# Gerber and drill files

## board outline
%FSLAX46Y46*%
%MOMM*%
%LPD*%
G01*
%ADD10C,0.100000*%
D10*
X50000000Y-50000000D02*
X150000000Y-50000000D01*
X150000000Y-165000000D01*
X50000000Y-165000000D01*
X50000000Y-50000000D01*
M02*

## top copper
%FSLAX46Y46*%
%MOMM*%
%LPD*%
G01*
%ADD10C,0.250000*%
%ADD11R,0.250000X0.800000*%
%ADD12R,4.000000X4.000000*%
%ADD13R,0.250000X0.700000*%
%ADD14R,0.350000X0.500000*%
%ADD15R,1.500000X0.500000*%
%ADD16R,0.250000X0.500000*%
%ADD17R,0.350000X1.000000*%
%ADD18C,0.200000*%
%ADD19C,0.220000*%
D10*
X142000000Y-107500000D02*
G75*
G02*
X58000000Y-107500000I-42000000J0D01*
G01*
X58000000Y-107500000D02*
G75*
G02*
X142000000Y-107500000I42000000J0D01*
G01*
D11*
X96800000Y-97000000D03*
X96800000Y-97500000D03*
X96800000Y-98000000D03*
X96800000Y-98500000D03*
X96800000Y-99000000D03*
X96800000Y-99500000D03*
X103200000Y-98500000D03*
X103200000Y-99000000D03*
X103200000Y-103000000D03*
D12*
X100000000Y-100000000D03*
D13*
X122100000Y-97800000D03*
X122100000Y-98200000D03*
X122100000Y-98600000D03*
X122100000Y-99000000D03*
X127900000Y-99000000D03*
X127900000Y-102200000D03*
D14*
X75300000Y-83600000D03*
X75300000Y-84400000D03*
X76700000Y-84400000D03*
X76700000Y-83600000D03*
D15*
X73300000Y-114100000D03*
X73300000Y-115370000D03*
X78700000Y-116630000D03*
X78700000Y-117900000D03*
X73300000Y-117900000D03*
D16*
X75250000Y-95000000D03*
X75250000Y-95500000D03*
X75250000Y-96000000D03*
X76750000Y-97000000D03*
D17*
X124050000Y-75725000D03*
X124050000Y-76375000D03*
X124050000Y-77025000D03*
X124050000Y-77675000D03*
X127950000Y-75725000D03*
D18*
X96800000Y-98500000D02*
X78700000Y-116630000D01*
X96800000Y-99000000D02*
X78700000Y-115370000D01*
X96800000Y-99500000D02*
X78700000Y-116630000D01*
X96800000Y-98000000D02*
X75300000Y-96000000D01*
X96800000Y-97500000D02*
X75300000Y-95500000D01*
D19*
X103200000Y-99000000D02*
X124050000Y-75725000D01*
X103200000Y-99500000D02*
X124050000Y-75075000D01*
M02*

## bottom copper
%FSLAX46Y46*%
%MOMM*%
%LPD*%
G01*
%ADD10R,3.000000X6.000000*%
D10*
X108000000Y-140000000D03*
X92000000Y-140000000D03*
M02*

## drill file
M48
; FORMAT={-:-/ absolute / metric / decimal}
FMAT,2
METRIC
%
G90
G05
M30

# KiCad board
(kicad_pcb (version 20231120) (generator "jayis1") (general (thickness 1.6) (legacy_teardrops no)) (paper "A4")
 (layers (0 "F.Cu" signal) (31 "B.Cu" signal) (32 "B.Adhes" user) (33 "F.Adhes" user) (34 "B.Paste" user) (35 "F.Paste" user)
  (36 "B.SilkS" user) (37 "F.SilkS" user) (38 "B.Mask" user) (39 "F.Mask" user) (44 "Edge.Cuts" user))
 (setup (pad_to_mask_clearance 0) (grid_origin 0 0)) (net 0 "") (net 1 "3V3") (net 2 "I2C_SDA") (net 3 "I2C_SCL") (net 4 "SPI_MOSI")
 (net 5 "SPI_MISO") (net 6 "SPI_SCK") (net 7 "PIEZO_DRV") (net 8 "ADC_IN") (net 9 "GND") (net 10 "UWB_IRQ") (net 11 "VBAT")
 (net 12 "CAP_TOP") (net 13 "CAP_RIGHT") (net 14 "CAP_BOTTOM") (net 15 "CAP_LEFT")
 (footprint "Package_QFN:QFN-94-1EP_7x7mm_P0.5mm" (layer "F.Cu") (at 100 100) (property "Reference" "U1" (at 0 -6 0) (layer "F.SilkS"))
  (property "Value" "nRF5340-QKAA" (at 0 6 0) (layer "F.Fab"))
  (pad "1" smd rect (at -3.2 -3 0) (size 0.25 0.8) (layers "F.Cu" "F.Mask" "F.Paste") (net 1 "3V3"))
  (pad "2" smd rect (at -3.2 -2.5 0) (size 0.25 0.8) (layers "F.Cu" "F.Mask" "F.Paste") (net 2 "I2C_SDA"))
  (pad "3" smd rect (at -3.2 -2.0 0) (size 0.25 0.8) (layers "F.Cu" "F.Mask" "F.Paste") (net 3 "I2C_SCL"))
  (pad "4" smd rect (at -3.2 -1.5 0) (size 0.25 0.8) (layers "F.Cu" "F.Mask" "F.Paste") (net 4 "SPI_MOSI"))
  (pad "5" smd rect (at -3.2 -1.0 0) (size 0.25 0.8) (layers "F.Cu" "F.Mask" "F.Paste") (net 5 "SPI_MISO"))
  (pad "6" smd rect (at -3.2 -0.5 0) (size 0.25 0.8) (layers "F.Cu" "F.Mask" "F.Paste") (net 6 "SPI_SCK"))
  (pad "21" smd rect (at 3.2 -1.5 180) (size 0.25 0.8) (layers "F.Cu" "F.Mask" "F.Paste") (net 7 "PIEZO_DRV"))
  (pad "22" smd rect (at 3.2 -1.0 180) (size 0.25 0.8) (layers "F.Cu" "F.Mask" "F.Paste") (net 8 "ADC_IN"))
  (pad "47" smd rect (at 3.2 3.0 180) (size 0.25 0.8) (layers "F.Cu" "F.Mask" "F.Paste") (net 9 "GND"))
  (pad "EP" smd rect (at 0 0 0) (size 4 4) (layers "F.Cu" "F.Mask") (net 9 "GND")))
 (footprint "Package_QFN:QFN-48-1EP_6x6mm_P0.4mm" (layer "F.Cu") (at 125 100) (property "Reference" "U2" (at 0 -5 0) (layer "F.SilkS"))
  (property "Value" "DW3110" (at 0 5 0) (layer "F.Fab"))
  (pad "1" smd rect (at -2.9 -2.2 0) (size 0.25 0.7) (layers "F.Cu" "F.Mask" "F.Paste") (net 1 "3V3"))
  (pad "2" smd rect (at -2.9 -1.8 0) (size 0.25 0.7) (layers "F.Cu" "F.Mask" "F.Paste") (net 4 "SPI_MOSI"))
  (pad "3" smd rect (at -2.9 -1.4 0) (size 0.25 0.7) (layers "F.Cu" "F.Mask" "F.Paste") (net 5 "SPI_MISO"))
  (pad "4" smd rect (at -2.9 -1.0 0) (size 0.25 0.7) (layers "F.Cu" "F.Mask" "F.Paste") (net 6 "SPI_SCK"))
  (pad "10" smd rect (at 2.9 -1.0 180) (size 0.25 0.7) (layers "F.Cu" "F.Mask" "F.Paste") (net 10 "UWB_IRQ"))
  (pad "48" smd rect (at 2.9 2.2 180) (size 0.25 0.7) (layers "F.Cu" "F.Mask" "F.Paste") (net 9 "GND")))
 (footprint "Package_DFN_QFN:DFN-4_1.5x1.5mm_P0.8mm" (layer "F.Cu") (at 76 84) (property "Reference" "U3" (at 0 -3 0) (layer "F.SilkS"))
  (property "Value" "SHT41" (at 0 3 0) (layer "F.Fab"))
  (pad "1" smd rect (at -0.7 -0.4 0) (size 0.35 0.5) (layers "F.Cu" "F.Mask" "F.Paste") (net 1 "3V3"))
  (pad "2" smd rect (at -0.7 0.4 0) (size 0.35 0.5) (layers "F.Cu" "F.Mask" "F.Paste") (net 2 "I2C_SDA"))
  (pad "3" smd rect (at 0.7 0.4 0) (size 0.35 0.5) (layers "F.Cu" "F.Mask" "F.Paste") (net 3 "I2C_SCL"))
  (pad "4" smd rect (at 0.7 -0.4 0) (size 0.35 0.5) (layers "F.Cu" "F.Mask" "F.Paste") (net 9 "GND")))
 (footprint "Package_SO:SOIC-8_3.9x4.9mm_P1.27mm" (layer "F.Cu") (at 76 116) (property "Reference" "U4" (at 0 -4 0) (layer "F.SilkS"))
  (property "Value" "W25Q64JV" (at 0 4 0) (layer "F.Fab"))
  (pad "1" smd rect (at -2.7 -1.9 0) (size 1.5 0.5) (layers "F.Cu" "F.Mask" "F.Paste") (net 4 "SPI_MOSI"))
  (pad "2" smd rect (at -2.7 -0.63 0) (size 1.5 0.5) (layers "F.Cu" "F.Mask" "F.Paste") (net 5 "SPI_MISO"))
  (pad "6" smd rect (at 2.7 0.63 0) (size 1.5 0.5) (layers "F.Cu" "F.Mask" "F.Paste") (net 6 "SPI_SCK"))
  (pad "8" smd rect (at 2.7 1.9 0) (size 1.5 0.5) (layers "F.Cu" "F.Mask" "F.Paste") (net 1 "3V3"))
  (pad "4" smd rect (at -2.7 1.9 0) (size 1.5 0.5) (layers "F.Cu" "F.Mask" "F.Paste") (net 9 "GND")))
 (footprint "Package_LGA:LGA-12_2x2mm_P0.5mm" (layer "F.Cu") (at 76 96) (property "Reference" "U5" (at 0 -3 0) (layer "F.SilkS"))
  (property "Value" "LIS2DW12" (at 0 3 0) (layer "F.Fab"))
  (pad "1" smd rect (at -0.75 -1.0 0) (size 0.25 0.5) (layers "F.Cu" "F.Mask" "F.Paste") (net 1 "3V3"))
  (pad "2" smd rect (at -0.75 -0.5 0) (size 0.25 0.5) (layers "F.Cu" "F.Mask" "F.Paste") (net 3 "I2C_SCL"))
  (pad "3" smd rect (at -0.75 0.0 0) (size 0.25 0.5) (layers "F.Cu" "F.Mask" "F.Paste") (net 2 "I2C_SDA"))
  (pad "12" smd rect (at 0.75 1.0 0) (size 0.25 0.5) (layers "F.Cu" "F.Mask" "F.Paste") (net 9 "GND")))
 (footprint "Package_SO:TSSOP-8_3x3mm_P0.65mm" (layer "F.Cu") (at 126 78) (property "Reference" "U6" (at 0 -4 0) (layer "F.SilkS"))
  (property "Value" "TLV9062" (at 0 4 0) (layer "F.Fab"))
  (pad "1" smd rect (at -1.95 -2.275 0) (size 0.35 1.0) (layers "F.Cu" "F.Mask" "F.Paste") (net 8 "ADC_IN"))
  (pad "2" smd rect (at -1.95 -1.625 0) (size 0.35 1.0) (layers "F.Cu" "F.Mask" "F.Paste") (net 9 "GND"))
  (pad "3" smd rect (at -1.95 -0.975 0) (size 0.35 1.0) (layers "F.Cu" "F.Mask" "F.Paste") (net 7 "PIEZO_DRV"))
  (pad "4" smd rect (at -1.95 -0.325 0) (size 0.35 1.0) (layers "F.Cu" "F.Mask" "F.Paste") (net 9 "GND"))
  (pad "8" smd rect (at 1.95 -2.275 0) (size 0.35 1.0) (layers "F.Cu" "F.Mask" "F.Paste") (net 1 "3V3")))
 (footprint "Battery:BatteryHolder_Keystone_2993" (layer "B.Cu") (at 100 140 180) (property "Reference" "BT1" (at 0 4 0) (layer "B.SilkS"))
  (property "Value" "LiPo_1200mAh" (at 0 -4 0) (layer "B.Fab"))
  (pad "1" smd rect (at -8 0 180) (size 3 6) (layers "B.Cu" "B.Mask") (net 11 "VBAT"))
  (pad "2" smd rect (at 8 0 180) (size 3 6) (layers "B.Cu" "B.Mask") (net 9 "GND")))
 (segment (start 96.8 98.5) (end 78.7 116.63) (width 0.2) (layer "F.Cu") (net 4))
 (segment (start 96.8 99.0) (end 78.7 115.37) (width 0.2) (layer "F.Cu") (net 5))
 (segment (start 96.8 99.5) (end 78.7 116.63) (width 0.2) (layer "F.Cu") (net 6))
 (segment (start 96.8 98.0) (end 75.3 96.0) (width 0.2) (layer "F.Cu") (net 2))
 (segment (start 96.8 97.5) (end 75.3 95.5) (width 0.2) (layer "F.Cu") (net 3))
 (segment (start 103.2 99.0) (end 124.05 75.725) (width 0.22) (layer "F.Cu") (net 7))
 (segment (start 103.2 99.5) (end 124.05 75.075) (width 0.22) (layer "F.Cu") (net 8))
 (gr_rect (start 50 50) (end 150 165) (stroke (width 0.1) (type default)) (fill no) (layer "Edge.Cuts"))
 (gr_circle (center 100 107.5) (end 142 107.5) (stroke (width 0.25) (type default)) (fill no) (layer "F.Cu")))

